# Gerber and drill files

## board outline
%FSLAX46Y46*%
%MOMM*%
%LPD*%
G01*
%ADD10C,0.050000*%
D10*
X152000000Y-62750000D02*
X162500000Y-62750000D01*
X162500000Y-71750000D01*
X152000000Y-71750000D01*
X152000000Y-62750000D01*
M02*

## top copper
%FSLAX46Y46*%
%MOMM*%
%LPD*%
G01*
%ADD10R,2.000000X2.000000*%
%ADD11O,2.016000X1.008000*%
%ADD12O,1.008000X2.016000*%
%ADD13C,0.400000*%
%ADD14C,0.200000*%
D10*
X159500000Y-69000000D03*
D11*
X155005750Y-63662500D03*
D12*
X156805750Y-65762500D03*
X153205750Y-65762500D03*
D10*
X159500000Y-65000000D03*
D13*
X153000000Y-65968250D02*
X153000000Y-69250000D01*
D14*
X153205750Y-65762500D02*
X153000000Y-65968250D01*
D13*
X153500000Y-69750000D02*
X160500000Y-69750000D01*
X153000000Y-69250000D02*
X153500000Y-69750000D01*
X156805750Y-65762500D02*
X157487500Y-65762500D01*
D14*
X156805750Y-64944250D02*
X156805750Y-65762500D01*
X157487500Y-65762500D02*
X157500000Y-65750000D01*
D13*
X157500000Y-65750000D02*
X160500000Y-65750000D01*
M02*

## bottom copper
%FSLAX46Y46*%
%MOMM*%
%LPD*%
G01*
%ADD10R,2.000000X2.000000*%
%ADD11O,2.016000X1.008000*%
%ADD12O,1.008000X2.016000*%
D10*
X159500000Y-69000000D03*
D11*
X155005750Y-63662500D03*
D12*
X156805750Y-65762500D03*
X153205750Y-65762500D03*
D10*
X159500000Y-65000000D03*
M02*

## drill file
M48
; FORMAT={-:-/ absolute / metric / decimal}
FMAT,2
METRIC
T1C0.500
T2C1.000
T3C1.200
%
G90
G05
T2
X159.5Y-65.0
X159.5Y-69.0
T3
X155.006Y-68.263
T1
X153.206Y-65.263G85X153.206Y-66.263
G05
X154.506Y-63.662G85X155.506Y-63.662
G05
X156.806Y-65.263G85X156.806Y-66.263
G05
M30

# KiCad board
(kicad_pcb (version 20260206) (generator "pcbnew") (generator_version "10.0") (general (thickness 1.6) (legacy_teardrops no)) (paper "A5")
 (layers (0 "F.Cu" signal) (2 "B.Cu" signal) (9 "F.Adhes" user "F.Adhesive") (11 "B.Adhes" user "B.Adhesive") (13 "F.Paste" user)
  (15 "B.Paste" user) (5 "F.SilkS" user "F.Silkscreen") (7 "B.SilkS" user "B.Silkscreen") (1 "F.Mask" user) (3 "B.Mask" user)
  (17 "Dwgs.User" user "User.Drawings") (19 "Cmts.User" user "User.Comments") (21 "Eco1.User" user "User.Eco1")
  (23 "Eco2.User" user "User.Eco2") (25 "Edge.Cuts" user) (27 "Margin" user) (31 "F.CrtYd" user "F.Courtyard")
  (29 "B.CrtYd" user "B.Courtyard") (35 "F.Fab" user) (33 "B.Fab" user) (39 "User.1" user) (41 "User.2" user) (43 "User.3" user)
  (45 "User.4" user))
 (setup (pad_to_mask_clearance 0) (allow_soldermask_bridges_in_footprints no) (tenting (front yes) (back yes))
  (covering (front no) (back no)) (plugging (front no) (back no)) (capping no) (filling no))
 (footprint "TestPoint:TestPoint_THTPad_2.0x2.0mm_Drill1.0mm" (layer "F.Cu") (at 159.5 69)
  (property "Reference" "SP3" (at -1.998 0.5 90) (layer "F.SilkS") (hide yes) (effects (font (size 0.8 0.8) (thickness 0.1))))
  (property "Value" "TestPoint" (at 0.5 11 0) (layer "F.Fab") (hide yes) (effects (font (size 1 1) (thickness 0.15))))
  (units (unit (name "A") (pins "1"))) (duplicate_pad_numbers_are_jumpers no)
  (pad "1" thru_hole rect (at 0 0) (size 2 2) (drill 1) (layers "*.Cu" "*.Mask") (remove_unused_layers no) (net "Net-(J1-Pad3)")))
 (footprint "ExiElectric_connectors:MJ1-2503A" (layer "F.Cu") (at 155.00575 68.2625)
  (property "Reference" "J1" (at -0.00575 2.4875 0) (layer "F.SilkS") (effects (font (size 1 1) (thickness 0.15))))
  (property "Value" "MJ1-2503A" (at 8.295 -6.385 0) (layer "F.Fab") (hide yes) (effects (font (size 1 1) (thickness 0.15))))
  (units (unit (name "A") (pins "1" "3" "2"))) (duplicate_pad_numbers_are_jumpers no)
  (pad "" np_thru_hole circle (at 0 0) (size 1.2 1.2) (drill 1.2) (layers "*.Cu" "*.Mask"))
  (pad "1" thru_hole oval (at 0 -4.6) (size 2.016 1.008) (drill oval 1.5 0.5) (layers "*.Cu" "*.Mask") (remove_unused_layers no)
   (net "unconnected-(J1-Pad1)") (solder_mask_margin 0.102))
  (pad "2" thru_hole oval (at 1.8 -2.5) (size 1.008 2.016) (drill oval 0.5 1.5) (layers "*.Cu" "*.Mask") (remove_unused_layers no)
   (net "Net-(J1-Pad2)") (solder_mask_margin 0.102))
  (pad "3" thru_hole oval (at -1.8 -2.5) (size 1.008 2.016) (drill oval 0.5 1.5) (layers "*.Cu" "*.Mask") (remove_unused_layers no)
   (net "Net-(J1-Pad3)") (solder_mask_margin 0.102)))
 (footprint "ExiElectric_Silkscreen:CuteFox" (layer "F.Cu") (at 155 66)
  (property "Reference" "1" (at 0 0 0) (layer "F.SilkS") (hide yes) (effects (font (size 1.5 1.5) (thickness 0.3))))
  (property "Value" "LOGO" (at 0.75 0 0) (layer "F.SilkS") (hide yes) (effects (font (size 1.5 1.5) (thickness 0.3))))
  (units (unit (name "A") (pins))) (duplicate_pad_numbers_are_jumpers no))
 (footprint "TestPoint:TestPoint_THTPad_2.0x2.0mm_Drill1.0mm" (layer "F.Cu") (at 159.5 65)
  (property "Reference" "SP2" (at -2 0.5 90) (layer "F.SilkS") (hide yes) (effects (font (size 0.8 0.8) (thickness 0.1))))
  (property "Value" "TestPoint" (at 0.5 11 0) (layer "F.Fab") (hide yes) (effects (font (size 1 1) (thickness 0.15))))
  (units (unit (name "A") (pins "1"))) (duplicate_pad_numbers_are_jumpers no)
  (pad "1" thru_hole rect (at 0 0) (size 2 2) (drill 1) (layers "*.Cu" "*.Mask") (remove_unused_layers no) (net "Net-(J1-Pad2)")))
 (gr_rect (start 152 62.75) (end 162.5 71.75) (stroke (width 0.05) (type default)) (fill no) (layer "Edge.Cuts"))
 (segment (start 153 65.96825) (end 153 69.25) (width 0.4) (layer "F.Cu") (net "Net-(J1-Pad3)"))
 (segment (start 153.20575 65.7625) (end 153 65.96825) (width 0.2) (layer "F.Cu") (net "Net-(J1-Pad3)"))
 (segment (start 153.5 69.75) (end 160.5 69.75) (width 0.4) (layer "F.Cu") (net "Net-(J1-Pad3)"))
 (segment (start 153 69.25) (end 153.5 69.75) (width 0.4) (layer "F.Cu") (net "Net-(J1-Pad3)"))
 (segment (start 156.80575 65.7625) (end 157.4875 65.7625) (width 0.4) (layer "F.Cu") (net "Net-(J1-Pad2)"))
 (segment (start 156.80575 64.94425) (end 156.80575 65.7625) (width 0.2) (layer "F.Cu") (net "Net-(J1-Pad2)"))
 (segment (start 157.4875 65.7625) (end 157.5 65.75) (width 0.2) (layer "F.Cu") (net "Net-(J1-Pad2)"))
 (segment (start 157.5 65.75) (end 160.5 65.75) (width 0.4) (layer "F.Cu") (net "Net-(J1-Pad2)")))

